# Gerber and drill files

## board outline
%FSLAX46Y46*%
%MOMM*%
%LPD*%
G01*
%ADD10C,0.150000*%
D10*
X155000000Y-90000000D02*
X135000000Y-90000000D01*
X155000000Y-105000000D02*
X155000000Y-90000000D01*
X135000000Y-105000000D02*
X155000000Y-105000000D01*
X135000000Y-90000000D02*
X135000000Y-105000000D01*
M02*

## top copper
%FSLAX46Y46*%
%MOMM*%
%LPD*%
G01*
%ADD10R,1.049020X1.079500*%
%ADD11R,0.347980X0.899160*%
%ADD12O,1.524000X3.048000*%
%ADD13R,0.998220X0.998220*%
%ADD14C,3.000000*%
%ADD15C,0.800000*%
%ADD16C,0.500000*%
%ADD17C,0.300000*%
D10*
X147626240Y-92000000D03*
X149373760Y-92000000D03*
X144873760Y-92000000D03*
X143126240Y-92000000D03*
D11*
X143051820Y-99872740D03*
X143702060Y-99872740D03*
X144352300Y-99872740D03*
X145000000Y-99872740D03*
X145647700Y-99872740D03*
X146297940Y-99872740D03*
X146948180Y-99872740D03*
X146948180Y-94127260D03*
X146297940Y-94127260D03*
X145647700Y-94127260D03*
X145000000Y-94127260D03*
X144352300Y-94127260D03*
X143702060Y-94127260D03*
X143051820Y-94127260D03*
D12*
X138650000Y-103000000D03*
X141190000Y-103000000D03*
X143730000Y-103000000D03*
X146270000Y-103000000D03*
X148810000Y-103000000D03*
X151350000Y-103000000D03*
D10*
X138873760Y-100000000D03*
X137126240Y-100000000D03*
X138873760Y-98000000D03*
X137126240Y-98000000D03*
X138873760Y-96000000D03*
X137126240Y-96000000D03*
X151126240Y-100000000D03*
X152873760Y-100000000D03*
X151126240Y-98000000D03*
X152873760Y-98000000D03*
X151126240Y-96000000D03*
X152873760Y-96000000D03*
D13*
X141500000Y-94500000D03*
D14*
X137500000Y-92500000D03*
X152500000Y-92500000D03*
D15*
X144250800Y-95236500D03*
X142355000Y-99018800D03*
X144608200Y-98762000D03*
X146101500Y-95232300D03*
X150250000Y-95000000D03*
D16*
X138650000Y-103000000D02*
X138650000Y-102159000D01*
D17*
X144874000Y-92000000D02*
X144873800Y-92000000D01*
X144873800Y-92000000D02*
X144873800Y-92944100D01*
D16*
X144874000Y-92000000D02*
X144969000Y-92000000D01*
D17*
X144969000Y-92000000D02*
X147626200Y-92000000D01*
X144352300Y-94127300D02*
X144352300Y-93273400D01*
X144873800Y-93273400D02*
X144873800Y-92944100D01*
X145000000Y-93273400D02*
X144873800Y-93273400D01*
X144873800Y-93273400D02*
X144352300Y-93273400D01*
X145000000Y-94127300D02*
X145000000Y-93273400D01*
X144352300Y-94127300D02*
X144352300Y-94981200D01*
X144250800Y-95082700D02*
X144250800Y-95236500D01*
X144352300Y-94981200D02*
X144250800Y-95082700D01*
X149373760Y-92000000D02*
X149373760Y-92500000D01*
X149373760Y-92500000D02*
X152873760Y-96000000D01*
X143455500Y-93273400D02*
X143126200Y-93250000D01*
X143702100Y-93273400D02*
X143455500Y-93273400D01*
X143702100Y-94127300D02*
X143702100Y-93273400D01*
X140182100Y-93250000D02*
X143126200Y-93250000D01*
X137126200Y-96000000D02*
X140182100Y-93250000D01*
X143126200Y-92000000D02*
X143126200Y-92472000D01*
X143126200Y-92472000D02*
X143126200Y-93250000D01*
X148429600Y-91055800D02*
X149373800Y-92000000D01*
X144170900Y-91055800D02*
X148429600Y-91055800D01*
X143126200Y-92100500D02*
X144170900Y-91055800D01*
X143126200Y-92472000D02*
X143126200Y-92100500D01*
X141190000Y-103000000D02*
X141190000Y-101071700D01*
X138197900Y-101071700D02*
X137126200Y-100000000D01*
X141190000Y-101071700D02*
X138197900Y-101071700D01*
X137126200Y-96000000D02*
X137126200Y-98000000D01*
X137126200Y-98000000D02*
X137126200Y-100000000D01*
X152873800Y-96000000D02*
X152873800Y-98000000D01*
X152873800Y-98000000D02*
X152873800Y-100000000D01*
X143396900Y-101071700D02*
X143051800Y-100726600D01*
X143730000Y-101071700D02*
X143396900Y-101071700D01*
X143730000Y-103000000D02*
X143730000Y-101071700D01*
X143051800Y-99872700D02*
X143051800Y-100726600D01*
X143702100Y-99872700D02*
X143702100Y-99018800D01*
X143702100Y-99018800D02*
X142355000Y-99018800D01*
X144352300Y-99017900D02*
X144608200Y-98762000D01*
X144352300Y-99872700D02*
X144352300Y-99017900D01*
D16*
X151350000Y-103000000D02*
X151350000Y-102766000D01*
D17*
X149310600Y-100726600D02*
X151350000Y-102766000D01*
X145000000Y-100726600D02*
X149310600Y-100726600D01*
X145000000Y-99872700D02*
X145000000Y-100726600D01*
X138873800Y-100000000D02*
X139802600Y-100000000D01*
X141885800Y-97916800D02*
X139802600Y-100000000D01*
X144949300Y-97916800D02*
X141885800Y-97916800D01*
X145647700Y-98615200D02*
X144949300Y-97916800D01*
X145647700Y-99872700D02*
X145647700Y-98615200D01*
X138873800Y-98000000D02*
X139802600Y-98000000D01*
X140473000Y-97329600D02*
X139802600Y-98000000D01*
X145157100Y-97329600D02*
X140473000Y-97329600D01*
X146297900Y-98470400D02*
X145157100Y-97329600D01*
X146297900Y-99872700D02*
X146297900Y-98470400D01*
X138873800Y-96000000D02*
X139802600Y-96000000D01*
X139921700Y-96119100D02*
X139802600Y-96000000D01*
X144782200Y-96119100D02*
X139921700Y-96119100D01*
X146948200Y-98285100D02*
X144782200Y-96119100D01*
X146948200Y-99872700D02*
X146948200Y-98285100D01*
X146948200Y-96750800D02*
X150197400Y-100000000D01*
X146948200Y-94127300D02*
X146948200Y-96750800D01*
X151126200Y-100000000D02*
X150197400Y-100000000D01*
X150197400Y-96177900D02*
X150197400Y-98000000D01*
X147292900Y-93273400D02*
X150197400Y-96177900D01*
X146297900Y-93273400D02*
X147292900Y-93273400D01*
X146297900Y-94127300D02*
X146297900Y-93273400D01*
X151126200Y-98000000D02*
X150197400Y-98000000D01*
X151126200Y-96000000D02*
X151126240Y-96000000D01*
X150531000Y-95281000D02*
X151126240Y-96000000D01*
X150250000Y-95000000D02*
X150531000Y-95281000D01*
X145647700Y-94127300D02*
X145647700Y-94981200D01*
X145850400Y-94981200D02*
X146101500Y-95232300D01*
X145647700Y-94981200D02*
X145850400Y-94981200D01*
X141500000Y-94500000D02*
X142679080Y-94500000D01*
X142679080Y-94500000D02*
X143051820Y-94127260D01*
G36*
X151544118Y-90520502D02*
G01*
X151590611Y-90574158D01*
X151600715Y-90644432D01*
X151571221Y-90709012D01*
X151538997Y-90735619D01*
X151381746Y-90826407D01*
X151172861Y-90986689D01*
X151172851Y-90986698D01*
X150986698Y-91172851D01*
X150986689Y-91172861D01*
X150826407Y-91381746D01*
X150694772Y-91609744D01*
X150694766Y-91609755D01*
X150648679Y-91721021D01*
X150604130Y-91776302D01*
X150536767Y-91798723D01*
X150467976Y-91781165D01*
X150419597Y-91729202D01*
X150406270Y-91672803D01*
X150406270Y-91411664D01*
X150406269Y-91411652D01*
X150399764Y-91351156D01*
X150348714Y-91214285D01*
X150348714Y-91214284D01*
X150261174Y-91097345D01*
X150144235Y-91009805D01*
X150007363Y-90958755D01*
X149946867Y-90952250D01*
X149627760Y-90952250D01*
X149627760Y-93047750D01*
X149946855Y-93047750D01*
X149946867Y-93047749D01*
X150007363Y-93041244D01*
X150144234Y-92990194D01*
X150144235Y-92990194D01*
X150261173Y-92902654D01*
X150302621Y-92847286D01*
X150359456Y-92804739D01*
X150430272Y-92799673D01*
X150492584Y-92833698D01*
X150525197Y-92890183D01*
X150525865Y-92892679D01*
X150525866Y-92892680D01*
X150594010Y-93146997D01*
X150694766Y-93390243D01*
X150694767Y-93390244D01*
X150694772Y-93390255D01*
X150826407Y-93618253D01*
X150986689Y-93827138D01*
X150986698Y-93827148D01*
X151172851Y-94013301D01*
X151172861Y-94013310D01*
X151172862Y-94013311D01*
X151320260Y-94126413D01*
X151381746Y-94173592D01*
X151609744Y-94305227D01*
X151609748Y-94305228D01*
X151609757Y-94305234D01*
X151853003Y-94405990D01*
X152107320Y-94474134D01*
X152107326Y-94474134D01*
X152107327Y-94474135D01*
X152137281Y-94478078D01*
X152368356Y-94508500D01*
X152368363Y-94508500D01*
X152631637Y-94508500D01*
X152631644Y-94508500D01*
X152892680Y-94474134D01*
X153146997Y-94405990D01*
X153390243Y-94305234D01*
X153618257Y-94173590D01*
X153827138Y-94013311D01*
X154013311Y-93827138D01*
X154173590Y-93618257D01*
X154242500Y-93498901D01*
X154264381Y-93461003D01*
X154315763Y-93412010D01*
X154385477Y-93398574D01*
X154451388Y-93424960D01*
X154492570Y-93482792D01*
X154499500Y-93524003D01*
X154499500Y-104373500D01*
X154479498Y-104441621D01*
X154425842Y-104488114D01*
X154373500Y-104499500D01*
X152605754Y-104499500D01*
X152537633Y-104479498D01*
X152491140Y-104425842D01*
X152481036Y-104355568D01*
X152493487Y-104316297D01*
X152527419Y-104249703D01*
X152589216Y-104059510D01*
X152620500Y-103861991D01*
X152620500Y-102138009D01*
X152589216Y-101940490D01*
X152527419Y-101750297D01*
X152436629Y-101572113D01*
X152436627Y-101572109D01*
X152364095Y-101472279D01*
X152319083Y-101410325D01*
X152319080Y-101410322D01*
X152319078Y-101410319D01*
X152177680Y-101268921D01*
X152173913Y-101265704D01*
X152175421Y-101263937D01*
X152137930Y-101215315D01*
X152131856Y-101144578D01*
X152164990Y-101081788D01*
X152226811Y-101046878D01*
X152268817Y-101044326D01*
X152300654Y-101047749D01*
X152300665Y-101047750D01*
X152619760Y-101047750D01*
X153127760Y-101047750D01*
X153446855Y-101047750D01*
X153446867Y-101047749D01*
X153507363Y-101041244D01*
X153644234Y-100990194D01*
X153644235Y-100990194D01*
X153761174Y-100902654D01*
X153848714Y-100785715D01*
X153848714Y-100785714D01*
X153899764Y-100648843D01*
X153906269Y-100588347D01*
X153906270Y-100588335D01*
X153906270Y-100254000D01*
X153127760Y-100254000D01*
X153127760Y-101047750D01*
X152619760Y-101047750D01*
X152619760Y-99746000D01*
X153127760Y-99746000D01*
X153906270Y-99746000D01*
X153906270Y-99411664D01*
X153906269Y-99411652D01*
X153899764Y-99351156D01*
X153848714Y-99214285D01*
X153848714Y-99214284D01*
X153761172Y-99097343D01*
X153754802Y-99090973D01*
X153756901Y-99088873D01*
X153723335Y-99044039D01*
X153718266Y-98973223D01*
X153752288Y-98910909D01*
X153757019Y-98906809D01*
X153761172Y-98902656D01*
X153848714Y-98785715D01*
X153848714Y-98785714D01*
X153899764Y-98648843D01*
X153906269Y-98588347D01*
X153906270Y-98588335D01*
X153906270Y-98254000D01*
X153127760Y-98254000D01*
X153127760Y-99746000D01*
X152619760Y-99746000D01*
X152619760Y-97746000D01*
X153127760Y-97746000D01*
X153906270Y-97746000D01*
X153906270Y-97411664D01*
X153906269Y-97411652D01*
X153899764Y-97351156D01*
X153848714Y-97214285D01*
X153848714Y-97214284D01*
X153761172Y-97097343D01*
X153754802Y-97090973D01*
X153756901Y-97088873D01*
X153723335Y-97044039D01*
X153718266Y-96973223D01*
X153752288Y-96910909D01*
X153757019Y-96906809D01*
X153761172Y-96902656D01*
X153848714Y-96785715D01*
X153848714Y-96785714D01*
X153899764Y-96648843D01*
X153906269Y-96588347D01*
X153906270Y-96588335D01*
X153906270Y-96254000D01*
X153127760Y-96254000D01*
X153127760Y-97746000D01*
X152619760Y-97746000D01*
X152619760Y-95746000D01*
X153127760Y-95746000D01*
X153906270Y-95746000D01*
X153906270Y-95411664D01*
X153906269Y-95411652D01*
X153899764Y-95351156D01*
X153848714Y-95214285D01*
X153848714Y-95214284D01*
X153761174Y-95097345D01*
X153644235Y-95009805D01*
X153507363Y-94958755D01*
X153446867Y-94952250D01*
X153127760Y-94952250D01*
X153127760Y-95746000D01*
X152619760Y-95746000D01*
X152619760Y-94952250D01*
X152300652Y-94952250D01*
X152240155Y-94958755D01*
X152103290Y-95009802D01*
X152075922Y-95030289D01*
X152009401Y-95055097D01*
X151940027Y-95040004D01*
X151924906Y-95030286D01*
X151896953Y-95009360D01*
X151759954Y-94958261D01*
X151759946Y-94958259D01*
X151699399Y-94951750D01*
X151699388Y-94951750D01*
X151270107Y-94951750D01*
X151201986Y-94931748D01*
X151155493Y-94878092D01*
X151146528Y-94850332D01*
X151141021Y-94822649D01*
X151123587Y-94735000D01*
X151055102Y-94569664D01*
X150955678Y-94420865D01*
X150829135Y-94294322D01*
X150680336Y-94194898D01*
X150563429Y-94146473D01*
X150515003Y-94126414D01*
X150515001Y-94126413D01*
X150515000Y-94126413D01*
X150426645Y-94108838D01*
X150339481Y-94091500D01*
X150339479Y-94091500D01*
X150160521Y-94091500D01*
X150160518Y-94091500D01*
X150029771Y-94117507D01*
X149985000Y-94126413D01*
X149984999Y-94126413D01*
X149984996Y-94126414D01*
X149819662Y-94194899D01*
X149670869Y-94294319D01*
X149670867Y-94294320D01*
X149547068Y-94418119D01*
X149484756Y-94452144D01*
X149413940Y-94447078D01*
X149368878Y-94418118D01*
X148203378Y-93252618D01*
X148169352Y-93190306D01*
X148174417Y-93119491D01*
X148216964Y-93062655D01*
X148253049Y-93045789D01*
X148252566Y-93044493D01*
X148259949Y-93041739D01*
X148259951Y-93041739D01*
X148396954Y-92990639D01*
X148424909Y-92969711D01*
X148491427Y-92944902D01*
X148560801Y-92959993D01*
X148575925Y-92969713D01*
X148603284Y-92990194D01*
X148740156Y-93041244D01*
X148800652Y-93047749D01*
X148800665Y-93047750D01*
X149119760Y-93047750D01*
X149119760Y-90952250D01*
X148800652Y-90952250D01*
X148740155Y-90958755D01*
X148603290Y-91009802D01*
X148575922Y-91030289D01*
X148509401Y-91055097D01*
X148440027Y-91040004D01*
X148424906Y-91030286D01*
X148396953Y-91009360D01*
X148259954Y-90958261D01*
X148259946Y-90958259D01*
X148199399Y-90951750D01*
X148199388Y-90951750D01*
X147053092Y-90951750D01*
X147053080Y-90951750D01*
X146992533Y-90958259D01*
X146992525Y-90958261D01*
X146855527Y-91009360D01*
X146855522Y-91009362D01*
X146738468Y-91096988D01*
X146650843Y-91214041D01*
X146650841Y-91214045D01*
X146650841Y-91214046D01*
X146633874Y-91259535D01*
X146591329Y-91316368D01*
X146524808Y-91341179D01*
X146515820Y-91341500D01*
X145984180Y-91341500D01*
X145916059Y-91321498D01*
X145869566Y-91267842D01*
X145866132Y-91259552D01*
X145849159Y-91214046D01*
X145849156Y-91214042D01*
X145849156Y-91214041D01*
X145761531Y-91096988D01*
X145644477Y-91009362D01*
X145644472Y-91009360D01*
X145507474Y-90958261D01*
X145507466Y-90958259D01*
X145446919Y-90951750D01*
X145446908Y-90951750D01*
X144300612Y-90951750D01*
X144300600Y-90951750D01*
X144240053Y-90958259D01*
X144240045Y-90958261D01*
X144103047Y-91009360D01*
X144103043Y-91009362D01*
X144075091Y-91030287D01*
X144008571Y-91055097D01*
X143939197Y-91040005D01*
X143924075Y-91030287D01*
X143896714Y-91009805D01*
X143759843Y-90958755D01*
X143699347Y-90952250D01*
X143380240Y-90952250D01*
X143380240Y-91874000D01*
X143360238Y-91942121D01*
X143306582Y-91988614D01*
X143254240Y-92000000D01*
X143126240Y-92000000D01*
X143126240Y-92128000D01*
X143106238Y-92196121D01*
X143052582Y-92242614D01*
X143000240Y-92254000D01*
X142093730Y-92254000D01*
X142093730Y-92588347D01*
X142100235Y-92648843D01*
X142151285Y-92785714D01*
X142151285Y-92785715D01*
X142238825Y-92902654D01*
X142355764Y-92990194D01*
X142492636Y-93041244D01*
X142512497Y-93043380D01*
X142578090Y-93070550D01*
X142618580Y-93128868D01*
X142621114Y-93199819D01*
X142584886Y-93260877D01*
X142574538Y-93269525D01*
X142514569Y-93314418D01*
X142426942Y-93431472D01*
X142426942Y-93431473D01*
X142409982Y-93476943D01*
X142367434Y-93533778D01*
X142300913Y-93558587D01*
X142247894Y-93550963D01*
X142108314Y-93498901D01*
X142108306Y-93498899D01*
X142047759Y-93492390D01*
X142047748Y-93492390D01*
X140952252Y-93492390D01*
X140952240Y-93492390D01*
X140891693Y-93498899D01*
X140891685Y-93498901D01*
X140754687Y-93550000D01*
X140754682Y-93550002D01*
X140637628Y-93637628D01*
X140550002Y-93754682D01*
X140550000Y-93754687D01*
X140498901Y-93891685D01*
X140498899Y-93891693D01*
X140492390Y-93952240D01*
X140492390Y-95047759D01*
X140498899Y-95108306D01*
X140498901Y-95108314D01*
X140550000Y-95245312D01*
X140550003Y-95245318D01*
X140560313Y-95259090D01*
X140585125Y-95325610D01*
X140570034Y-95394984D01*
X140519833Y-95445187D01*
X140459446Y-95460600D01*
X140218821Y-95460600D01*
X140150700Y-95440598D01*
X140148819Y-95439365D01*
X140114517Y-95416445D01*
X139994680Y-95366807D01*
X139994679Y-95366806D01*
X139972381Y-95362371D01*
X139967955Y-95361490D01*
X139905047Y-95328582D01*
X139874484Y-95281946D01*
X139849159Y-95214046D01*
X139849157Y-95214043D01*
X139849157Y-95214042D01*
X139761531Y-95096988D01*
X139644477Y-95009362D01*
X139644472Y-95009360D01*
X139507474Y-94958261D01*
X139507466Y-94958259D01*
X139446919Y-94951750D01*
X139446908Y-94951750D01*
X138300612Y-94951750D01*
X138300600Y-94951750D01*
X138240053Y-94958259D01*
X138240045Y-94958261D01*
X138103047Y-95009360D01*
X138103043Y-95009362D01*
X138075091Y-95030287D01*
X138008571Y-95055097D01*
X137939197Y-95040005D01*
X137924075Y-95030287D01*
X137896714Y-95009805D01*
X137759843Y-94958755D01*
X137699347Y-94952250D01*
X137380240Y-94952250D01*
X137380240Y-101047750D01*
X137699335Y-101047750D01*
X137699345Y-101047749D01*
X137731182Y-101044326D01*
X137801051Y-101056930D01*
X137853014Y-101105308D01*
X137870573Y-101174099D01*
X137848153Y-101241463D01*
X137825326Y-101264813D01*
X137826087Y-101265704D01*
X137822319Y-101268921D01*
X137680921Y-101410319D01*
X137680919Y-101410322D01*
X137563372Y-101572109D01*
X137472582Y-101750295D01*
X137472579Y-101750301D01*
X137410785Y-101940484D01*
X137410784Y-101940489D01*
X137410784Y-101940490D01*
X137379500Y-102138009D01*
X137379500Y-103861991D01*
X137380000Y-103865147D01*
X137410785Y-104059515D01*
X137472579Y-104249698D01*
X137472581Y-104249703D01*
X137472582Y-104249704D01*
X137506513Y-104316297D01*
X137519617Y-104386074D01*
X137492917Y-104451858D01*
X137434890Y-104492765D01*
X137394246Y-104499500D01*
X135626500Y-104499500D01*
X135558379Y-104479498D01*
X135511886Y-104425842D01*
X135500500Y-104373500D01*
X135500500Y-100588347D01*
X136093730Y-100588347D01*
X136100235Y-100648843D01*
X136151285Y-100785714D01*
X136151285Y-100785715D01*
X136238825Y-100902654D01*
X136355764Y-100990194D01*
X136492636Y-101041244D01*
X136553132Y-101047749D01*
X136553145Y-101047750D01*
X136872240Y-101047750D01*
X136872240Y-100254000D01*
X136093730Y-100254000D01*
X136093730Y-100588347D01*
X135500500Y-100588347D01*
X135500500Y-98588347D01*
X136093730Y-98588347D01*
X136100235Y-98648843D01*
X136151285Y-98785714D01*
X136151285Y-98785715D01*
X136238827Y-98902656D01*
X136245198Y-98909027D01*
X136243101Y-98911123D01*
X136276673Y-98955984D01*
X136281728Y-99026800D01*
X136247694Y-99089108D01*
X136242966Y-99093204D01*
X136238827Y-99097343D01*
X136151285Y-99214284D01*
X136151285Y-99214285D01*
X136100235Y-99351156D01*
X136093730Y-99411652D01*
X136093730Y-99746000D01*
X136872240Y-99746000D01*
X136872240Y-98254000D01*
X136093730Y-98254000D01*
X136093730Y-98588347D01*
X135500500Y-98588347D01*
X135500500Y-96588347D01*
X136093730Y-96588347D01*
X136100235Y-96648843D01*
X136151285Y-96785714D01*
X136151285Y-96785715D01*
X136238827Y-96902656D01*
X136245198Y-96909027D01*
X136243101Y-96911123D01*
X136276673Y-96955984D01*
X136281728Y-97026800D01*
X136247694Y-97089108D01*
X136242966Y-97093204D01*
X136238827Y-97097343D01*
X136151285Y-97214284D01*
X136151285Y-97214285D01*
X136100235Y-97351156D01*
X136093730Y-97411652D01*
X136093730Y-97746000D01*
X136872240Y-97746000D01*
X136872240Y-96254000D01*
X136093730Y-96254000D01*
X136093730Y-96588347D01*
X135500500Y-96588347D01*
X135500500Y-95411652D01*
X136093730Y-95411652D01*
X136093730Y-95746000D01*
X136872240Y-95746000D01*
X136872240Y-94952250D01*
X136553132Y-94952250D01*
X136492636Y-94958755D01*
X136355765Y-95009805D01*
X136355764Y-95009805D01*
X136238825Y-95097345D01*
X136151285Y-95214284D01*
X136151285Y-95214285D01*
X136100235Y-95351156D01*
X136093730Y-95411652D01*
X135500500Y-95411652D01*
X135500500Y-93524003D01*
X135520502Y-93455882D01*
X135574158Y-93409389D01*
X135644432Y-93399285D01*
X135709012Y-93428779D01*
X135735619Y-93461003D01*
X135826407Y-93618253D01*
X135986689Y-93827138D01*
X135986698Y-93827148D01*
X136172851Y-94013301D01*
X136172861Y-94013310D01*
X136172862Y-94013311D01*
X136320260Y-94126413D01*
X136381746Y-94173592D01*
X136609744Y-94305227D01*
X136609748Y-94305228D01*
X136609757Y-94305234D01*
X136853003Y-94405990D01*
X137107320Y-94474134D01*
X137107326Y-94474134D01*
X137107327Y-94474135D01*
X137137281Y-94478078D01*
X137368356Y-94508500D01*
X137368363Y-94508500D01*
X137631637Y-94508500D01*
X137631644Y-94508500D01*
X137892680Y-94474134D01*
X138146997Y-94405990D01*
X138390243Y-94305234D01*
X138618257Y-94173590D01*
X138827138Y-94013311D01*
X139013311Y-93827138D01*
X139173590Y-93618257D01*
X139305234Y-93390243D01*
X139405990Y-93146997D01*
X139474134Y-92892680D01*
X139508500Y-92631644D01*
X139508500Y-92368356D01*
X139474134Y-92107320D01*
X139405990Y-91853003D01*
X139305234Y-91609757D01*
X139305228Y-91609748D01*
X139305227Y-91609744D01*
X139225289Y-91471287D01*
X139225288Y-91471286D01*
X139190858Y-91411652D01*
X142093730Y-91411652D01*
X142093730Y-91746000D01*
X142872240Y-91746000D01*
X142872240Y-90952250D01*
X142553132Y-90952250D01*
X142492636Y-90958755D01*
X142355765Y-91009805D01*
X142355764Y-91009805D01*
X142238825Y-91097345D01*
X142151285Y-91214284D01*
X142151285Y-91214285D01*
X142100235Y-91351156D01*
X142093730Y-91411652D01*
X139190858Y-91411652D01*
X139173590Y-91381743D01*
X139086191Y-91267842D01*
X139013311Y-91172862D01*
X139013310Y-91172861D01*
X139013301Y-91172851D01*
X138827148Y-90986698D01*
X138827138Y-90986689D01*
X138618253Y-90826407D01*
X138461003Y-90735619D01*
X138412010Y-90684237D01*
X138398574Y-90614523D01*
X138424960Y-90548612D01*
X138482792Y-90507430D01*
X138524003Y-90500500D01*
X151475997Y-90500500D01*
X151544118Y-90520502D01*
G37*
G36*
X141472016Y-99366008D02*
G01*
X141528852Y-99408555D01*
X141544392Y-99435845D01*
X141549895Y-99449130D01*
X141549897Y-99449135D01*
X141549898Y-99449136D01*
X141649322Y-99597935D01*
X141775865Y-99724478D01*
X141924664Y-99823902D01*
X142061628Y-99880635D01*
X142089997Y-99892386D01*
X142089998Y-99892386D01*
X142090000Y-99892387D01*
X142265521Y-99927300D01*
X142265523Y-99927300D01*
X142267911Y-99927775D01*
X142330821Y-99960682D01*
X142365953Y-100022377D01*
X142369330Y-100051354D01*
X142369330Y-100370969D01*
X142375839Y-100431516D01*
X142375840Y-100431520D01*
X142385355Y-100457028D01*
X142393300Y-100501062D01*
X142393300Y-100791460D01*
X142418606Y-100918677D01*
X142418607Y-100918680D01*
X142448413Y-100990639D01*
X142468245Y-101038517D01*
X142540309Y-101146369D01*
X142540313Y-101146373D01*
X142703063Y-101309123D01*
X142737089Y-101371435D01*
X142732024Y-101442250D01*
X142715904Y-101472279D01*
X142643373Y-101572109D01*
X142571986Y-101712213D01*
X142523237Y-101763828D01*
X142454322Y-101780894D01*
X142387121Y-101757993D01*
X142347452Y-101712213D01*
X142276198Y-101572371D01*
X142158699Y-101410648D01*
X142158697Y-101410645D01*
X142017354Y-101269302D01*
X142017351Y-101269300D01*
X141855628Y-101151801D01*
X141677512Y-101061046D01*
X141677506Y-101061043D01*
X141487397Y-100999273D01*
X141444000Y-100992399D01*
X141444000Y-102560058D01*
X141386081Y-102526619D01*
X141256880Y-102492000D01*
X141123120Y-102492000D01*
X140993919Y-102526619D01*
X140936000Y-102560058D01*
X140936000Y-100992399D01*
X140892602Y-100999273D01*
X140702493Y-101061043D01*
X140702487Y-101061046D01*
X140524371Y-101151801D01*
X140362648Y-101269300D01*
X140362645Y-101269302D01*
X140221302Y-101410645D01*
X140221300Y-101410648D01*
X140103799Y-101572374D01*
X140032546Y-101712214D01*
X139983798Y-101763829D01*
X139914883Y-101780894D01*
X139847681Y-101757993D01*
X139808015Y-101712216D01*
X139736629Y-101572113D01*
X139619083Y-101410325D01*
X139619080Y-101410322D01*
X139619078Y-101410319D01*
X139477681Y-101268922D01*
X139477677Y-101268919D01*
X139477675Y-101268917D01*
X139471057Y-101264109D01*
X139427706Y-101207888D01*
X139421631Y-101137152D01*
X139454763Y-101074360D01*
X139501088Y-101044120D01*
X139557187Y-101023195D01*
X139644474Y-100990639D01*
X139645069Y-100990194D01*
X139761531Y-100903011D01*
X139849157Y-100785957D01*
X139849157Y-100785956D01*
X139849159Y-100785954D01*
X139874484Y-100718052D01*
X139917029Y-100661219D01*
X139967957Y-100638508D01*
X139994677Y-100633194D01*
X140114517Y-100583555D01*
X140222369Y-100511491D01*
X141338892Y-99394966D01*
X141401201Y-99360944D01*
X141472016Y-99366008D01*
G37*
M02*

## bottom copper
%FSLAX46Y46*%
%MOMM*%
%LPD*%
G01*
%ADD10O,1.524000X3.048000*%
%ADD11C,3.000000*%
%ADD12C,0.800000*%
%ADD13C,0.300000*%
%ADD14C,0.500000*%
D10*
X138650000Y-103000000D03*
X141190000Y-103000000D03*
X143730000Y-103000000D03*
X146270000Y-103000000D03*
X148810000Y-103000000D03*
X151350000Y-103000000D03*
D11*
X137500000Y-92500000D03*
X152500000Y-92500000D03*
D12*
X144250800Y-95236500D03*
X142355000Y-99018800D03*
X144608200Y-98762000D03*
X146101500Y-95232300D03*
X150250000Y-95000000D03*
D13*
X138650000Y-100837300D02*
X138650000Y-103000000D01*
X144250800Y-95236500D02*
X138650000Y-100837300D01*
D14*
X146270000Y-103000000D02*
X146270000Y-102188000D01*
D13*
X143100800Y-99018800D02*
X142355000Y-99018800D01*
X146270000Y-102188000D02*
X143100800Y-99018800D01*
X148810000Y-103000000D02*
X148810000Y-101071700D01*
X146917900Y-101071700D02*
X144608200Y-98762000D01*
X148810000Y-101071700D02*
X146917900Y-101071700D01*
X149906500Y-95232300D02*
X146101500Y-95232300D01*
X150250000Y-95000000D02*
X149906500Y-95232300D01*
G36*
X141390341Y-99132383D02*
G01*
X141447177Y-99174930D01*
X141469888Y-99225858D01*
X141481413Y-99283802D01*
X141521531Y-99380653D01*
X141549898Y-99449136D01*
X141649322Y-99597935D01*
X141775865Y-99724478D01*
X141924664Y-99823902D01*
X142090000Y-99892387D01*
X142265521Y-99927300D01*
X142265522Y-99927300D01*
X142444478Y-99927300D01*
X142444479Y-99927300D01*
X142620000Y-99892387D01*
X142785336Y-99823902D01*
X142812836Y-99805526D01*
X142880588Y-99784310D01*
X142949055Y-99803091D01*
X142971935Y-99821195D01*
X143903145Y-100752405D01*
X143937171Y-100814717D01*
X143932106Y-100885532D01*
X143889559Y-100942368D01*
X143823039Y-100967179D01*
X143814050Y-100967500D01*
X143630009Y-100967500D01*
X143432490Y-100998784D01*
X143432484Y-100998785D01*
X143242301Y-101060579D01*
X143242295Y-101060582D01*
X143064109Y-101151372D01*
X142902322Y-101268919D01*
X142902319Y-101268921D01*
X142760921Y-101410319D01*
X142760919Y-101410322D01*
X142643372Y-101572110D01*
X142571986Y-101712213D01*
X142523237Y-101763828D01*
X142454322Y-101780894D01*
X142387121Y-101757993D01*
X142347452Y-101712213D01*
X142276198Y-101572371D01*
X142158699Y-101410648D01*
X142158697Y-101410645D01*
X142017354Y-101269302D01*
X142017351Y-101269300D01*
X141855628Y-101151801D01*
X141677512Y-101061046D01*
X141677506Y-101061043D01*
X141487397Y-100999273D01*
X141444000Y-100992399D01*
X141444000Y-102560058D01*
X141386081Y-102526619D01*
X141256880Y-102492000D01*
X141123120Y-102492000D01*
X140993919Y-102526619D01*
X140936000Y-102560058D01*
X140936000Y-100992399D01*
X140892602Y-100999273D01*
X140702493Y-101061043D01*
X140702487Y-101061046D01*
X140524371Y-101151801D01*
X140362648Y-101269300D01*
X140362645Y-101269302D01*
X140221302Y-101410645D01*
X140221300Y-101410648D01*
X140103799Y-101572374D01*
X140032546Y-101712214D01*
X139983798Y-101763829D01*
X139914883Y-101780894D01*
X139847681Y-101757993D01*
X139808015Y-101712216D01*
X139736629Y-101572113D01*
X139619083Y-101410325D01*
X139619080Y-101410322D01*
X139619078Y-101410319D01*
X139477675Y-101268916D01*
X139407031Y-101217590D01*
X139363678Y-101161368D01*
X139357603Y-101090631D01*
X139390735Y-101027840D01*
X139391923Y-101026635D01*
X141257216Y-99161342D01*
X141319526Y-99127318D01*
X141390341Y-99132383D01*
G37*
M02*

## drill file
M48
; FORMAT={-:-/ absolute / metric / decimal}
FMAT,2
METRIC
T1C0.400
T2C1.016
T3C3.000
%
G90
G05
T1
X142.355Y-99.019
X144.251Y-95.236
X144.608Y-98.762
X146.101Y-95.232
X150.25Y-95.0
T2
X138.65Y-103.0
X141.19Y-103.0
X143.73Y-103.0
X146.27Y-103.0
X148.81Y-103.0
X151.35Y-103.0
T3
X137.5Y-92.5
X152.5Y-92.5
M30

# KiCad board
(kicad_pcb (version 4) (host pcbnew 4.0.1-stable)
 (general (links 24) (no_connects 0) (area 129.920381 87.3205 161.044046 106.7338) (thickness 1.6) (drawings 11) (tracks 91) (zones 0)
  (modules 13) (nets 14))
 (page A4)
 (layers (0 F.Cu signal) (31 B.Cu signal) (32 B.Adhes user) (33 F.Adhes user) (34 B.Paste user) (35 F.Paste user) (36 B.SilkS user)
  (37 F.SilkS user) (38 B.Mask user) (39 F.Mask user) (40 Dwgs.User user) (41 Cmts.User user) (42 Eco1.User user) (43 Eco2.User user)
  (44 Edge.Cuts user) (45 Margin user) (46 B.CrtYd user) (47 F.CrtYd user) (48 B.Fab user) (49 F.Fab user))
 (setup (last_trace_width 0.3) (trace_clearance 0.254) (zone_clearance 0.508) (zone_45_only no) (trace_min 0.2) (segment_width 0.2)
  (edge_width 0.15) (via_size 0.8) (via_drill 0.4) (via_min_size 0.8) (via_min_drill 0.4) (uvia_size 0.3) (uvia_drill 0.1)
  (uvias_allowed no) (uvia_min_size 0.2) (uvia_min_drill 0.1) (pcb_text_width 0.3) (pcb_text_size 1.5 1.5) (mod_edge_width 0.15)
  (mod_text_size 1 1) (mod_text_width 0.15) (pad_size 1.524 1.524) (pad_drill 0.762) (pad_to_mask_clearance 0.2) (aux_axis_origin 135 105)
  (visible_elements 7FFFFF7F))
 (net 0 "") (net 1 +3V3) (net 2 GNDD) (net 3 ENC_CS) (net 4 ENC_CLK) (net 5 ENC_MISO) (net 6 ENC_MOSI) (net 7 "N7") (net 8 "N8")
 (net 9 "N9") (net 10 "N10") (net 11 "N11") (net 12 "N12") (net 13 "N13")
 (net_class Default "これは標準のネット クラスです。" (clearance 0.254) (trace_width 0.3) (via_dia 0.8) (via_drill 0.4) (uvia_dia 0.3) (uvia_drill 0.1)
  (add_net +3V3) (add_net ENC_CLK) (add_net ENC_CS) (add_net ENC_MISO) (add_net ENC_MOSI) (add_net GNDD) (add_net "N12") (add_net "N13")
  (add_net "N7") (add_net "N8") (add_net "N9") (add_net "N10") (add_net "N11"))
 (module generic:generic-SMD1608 (layer F.Cu) (at 148.5 92)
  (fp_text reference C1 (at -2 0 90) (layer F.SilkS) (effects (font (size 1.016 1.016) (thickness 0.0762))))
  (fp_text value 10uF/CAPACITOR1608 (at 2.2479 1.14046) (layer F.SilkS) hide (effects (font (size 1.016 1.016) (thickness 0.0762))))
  (pad 1 smd rect (at -0.87376 0) (size 1.04902 1.0795) (layers F.Cu F.Paste F.Mask) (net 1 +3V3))
  (pad 2 smd rect (at 0.87376 0) (size 1.04902 1.0795) (layers F.Cu F.Paste F.Mask) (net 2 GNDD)))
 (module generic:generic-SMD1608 (layer F.Cu) (at 144 92 180)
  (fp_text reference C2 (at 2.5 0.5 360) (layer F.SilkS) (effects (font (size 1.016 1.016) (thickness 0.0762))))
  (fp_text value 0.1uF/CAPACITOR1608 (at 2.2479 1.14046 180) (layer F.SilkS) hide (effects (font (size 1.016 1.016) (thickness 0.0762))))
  (pad 1 smd rect (at -0.87376 0 180) (size 1.04902 1.0795) (layers F.Cu F.Paste F.Mask) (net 1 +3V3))
  (pad 2 smd rect (at 0.87376 0 180) (size 1.04902 1.0795) (layers F.Cu F.Paste F.Mask) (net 2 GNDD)))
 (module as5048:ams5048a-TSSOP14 (layer F.Cu) (at 145 97 90)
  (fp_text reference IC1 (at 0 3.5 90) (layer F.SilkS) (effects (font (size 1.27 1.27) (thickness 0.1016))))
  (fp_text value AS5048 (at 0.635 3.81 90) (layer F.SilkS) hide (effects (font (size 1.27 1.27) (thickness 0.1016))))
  (pad 1 smd rect (at -2.87274 -1.94818 90) (size 0.89916 0.34798) (layers F.Cu F.Paste F.Mask) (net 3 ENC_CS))
  (pad 2 smd rect (at -2.87274 -1.29794 90) (size 0.89916 0.34798) (layers F.Cu F.Paste F.Mask) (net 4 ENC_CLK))
  (pad 3 smd rect (at -2.87274 -0.6477 90) (size 0.89916 0.34798) (layers F.Cu F.Paste F.Mask) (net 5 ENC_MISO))
  (pad 4 smd rect (at -2.87274 0 90) (size 0.89916 0.34798) (layers F.Cu F.Paste F.Mask) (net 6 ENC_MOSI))
  (pad 5 smd rect (at -2.87274 0.6477 90) (size 0.89916 0.34798) (layers F.Cu F.Paste F.Mask) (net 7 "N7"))
  (pad 6 smd rect (at -2.87274 1.29794 90) (size 0.89916 0.34798) (layers F.Cu F.Paste F.Mask) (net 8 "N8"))
  (pad 7 smd rect (at -2.87274 1.94818 90) (size 0.89916 0.34798) (layers F.Cu F.Paste F.Mask) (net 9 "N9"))
  (pad 8 smd rect (at 2.87274 1.94818 90) (size 0.89916 0.34798) (layers F.Cu F.Paste F.Mask) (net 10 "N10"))
  (pad 9 smd rect (at 2.87274 1.29794 90) (size 0.89916 0.34798) (layers F.Cu F.Paste F.Mask) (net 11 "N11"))
  (pad 10 smd rect (at 2.87274 0.6477 90) (size 0.89916 0.34798) (layers F.Cu F.Paste F.Mask) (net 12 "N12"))
  (pad 11 smd rect (at 2.87274 0 90) (size 0.89916 0.34798) (layers F.Cu F.Paste F.Mask) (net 1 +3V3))
  (pad 12 smd rect (at 2.87274 -0.6477 90) (size 0.89916 0.34798) (layers F.Cu F.Paste F.Mask) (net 1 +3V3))
  (pad 13 smd rect (at 2.87274 -1.29794 90) (size 0.89916 0.34798) (layers F.Cu F.Paste F.Mask) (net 2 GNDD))
  (pad 14 smd rect (at 2.87274 -1.94818 90) (size 0.89916 0.34798) (layers F.Cu F.Paste F.Mask) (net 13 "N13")))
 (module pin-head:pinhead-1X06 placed (layer F.Cu) (at 145 103)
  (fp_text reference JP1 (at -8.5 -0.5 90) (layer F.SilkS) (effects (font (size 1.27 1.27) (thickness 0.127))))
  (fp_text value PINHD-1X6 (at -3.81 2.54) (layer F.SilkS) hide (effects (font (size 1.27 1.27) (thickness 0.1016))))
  (pad 1 thru_hole oval (at -6.35 0 180) (size 1.524 3.048) (drill 1.016) (layers *.Cu F.Paste F.SilkS F.Mask) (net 1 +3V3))
  (pad 2 thru_hole oval (at -3.81 0 180) (size 1.524 3.048) (drill 1.016) (layers *.Cu F.Paste F.SilkS F.Mask) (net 2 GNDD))
  (pad 3 thru_hole oval (at -1.27 0 180) (size 1.524 3.048) (drill 1.016) (layers *.Cu F.Paste F.SilkS F.Mask) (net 3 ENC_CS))
  (pad 4 thru_hole oval (at 1.27 0 180) (size 1.524 3.048) (drill 1.016) (layers *.Cu F.Paste F.SilkS F.Mask) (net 4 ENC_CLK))
  (pad 5 thru_hole oval (at 3.81 0 180) (size 1.524 3.048) (drill 1.016) (layers *.Cu F.Paste F.SilkS F.Mask) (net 5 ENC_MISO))
  (pad 6 thru_hole oval (at 6.35 0 180) (size 1.524 3.048) (drill 1.016) (layers *.Cu F.Paste F.SilkS F.Mask) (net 6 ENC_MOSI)))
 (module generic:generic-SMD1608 (layer F.Cu) (at 138 100 180)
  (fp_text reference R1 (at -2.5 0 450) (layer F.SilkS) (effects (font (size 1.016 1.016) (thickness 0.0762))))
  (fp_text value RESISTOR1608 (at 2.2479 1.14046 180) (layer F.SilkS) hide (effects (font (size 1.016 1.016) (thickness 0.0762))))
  (pad 1 smd rect (at -0.87376 0 180) (size 1.04902 1.0795) (layers F.Cu F.Paste F.Mask) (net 7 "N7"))
  (pad 2 smd rect (at 0.87376 0 180) (size 1.04902 1.0795) (layers F.Cu F.Paste F.Mask) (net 2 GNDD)))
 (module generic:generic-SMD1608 (layer F.Cu) (at 138 98 180)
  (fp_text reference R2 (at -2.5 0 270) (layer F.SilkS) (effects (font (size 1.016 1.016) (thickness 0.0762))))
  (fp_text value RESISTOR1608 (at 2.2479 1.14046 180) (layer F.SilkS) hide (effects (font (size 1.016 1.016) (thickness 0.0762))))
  (pad 1 smd rect (at -0.87376 0 180) (size 1.04902 1.0795) (layers F.Cu F.Paste F.Mask) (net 8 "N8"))
  (pad 2 smd rect (at 0.87376 0 180) (size 1.04902 1.0795) (layers F.Cu F.Paste F.Mask) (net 2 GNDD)))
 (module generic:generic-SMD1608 (layer F.Cu) (at 138 96 180)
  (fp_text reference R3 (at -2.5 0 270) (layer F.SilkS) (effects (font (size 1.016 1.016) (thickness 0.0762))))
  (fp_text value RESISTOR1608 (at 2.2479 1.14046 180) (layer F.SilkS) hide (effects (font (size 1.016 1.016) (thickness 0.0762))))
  (pad 1 smd rect (at -0.87376 0 180) (size 1.04902 1.0795) (layers F.Cu F.Paste F.Mask) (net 9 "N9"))
  (pad 2 smd rect (at 0.87376 0 180) (size 1.04902 1.0795) (layers F.Cu F.Paste F.Mask) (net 2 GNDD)))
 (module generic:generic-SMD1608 (layer F.Cu) (at 152 100)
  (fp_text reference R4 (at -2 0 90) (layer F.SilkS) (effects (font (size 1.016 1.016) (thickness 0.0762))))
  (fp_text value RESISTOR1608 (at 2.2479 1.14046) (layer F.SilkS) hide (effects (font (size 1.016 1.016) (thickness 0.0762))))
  (pad 1 smd rect (at -0.87376 0) (size 1.04902 1.0795) (layers F.Cu F.Paste F.Mask) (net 10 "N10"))
  (pad 2 smd rect (at 0.87376 0) (size 1.04902 1.0795) (layers F.Cu F.Paste F.Mask) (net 2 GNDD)))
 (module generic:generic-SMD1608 (layer F.Cu) (at 152 98)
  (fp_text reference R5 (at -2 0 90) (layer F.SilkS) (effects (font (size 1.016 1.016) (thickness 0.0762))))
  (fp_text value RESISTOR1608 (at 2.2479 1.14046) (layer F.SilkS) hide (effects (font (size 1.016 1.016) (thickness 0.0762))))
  (pad 1 smd rect (at -0.87376 0) (size 1.04902 1.0795) (layers F.Cu F.Paste F.Mask) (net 11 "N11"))
  (pad 2 smd rect (at 0.87376 0) (size 1.04902 1.0795) (layers F.Cu F.Paste F.Mask) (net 2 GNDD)))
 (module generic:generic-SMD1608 (layer F.Cu) (at 152 96)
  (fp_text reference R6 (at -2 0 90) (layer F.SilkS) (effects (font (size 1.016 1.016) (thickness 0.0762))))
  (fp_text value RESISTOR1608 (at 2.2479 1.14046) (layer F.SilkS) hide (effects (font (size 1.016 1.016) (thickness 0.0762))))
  (pad 1 smd rect (at -0.87376 0) (size 1.04902 1.0795) (layers F.Cu F.Paste F.Mask) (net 12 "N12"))
  (pad 2 smd rect (at 0.87376 0) (size 1.04902 1.0795) (layers F.Cu F.Paste F.Mask) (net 2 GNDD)))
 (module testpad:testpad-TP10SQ (layer F.Cu) (at 141 94.5)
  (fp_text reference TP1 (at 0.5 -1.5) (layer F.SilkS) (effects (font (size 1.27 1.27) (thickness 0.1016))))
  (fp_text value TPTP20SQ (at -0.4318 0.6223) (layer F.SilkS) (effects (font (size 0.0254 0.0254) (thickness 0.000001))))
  (pad TP smd rect (at 0.5 0) (size 0.99822 0.99822) (layers F.Cu F.Paste F.Mask) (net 13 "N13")))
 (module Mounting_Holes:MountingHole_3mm (layer F.Cu) (at 137.5 92.5)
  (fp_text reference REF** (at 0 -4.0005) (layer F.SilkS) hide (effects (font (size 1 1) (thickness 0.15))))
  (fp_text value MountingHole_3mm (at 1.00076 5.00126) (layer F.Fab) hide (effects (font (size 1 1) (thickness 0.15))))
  (pad 1 thru_hole circle (at 0 0) (size 3 3) (drill 3) (layers)))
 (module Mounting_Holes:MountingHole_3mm (layer F.Cu) (at 152.5 92.5)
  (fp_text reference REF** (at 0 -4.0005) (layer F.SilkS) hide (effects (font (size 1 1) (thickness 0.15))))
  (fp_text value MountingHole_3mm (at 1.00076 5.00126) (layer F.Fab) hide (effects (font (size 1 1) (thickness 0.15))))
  (pad 1 thru_hole circle (at 0 0) (size 3 3) (drill 3) (layers)))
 (gr_line (start 155 90) (end 135 90) (angle 90) (layer Edge.Cuts) (width 0.15))
 (gr_line (start 155 105) (end 155 90) (angle 90) (layer Edge.Cuts) (width 0.15))
 (gr_line (start 135 105) (end 155 105) (angle 90) (layer Edge.Cuts) (width 0.15))
 (gr_line (start 135 90) (end 135 105) (angle 90) (layer Edge.Cuts) (width 0.15))
 (via (at 144.2508 95.2365) (size 0.8) (layers F.Cu B.Cu) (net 1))
 (segment (start 138.65 103) (end 138.65 102.159) (width 0.5) (layer F.Cu) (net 1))
 (segment (start 144.874 92) (end 144.8738 92) (width 0.3) (layer F.Cu) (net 1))
 (segment (start 144.8738 92) (end 144.8738 92.9441) (width 0.3) (layer F.Cu) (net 1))
 (segment (start 144.874 92) (end 144.969 92) (width 0.5) (layer F.Cu) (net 1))
 (segment (start 144.969 92) (end 147.6262 92) (width 0.3) (layer F.Cu) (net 1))
 (segment (start 144.3523 94.1273) (end 144.3523 93.2734) (width 0.3) (layer F.Cu) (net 1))
 (segment (start 144.8738 93.2734) (end 144.8738 92.9441) (width 0.3) (layer F.Cu) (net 1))
 (segment (start 145 93.2734) (end 144.8738 93.2734) (width 0.3) (layer F.Cu) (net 1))
 (segment (start 144.8738 93.2734) (end 144.3523 93.2734) (width 0.3) (layer F.Cu) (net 1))
 (segment (start 145 94.1273) (end 145 93.2734) (width 0.3) (layer F.Cu) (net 1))
 (segment (start 144.3523 94.1273) (end 144.3523 94.9812) (width 0.3) (layer F.Cu) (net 1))
 (segment (start 144.2508 95.0827) (end 144.2508 95.2365) (width 0.3) (layer F.Cu) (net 1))
 (segment (start 144.3523 94.9812) (end 144.2508 95.0827) (width 0.3) (layer F.Cu) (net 1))
 (segment (start 138.65 100.8373) (end 138.65 103) (width 0.3) (layer B.Cu) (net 1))
 (segment (start 144.2508 95.2365) (end 138.65 100.8373) (width 0.3) (layer B.Cu) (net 1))
 (segment (start 149.37376 92) (end 149.37376 92.5) (width 0.3) (layer F.Cu) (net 2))
 (segment (start 149.37376 92.5) (end 152.87376 96) (width 0.3) (layer F.Cu) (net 2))
 (segment (start 143.4555 93.2734) (end 143.1262 93.25) (width 0.3) (layer F.Cu) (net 2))
 (segment (start 143.7021 93.2734) (end 143.4555 93.2734) (width 0.3) (layer F.Cu) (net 2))
 (segment (start 143.7021 94.1273) (end 143.7021 93.2734) (width 0.3) (layer F.Cu) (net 2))
 (segment (start 140.1821 93.25) (end 143.1262 93.25) (width 0.3) (layer F.Cu) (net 2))
 (segment (start 137.1262 96) (end 140.1821 93.25) (width 0.3) (layer F.Cu) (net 2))
 (segment (start 143.1262 92) (end 143.1262 92.472) (width 0.3) (layer F.Cu) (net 2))
 (segment (start 143.1262 92.472) (end 143.1262 93.25) (width 0.3) (layer F.Cu) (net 2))
 (segment (start 148.4296 91.0558) (end 149.3738 92) (width 0.3) (layer F.Cu) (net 2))
 (segment (start 144.1709 91.0558) (end 148.4296 91.0558) (width 0.3) (layer F.Cu) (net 2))
 (segment (start 143.1262 92.1005) (end 144.1709 91.0558) (width 0.3) (layer F.Cu) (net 2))
 (segment (start 143.1262 92.472) (end 143.1262 92.1005) (width 0.3) (layer F.Cu) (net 2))
 (segment (start 141.19 103) (end 141.19 101.0717) (width 0.3) (layer F.Cu) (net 2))
 (segment (start 138.1979 101.0717) (end 137.1262 100) (width 0.3) (layer F.Cu) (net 2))
 (segment (start 141.19 101.0717) (end 138.1979 101.0717) (width 0.3) (layer F.Cu) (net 2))
 (segment (start 137.1262 96) (end 137.1262 98) (width 0.3) (layer F.Cu) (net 2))
 (segment (start 137.1262 98) (end 137.1262 100) (width 0.3) (layer F.Cu) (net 2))
 (segment (start 152.8738 96) (end 152.8738 98) (width 0.3) (layer F.Cu) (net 2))
 (segment (start 152.8738 98) (end 152.8738 100) (width 0.3) (layer F.Cu) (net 2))
 (segment (start 143.3969 101.0717) (end 143.0518 100.7266) (width 0.3) (layer F.Cu) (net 3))
 (segment (start 143.73 101.0717) (end 143.3969 101.0717) (width 0.3) (layer F.Cu) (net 3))
 (segment (start 143.73 103) (end 143.73 101.0717) (width 0.3) (layer F.Cu) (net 3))
 (segment (start 143.0518 99.8727) (end 143.0518 100.7266) (width 0.3) (layer F.Cu) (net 3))
 (via (at 142.355 99.0188) (size 0.8) (layers F.Cu B.Cu) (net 4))
 (segment (start 146.27 103) (end 146.27 102.188) (width 0.5) (layer B.Cu) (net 4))
 (segment (start 143.7021 99.8727) (end 143.7021 99.0188) (width 0.3) (layer F.Cu) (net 4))
 (segment (start 143.1008 99.0188) (end 142.355 99.0188) (width 0.3) (layer B.Cu) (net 4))
 (segment (start 146.27 102.188) (end 143.1008 99.0188) (width 0.3) (layer B.Cu) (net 4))
 (segment (start 143.7021 99.0188) (end 142.355 99.0188) (width 0.3) (layer F.Cu) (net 4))
 (via (at 144.6082 98.762) (size 0.8) (layers F.Cu B.Cu) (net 5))
 (segment (start 148.81 103) (end 148.81 101.0717) (width 0.3) (layer B.Cu) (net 5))
 (segment (start 144.3523 99.0179) (end 144.6082 98.762) (width 0.3) (layer F.Cu) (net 5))
 (segment (start 144.3523 99.8727) (end 144.3523 99.0179) (width 0.3) (layer F.Cu) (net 5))
 (segment (start 146.9179 101.0717) (end 144.6082 98.762) (width 0.3) (layer B.Cu) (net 5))
 (segment (start 148.81 101.0717) (end 146.9179 101.0717) (width 0.3) (layer B.Cu) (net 5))
 (segment (start 151.35 103) (end 151.35 102.766) (width 0.5) (layer F.Cu) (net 6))
 (segment (start 149.3106 100.7266) (end 151.35 102.766) (width 0.3) (layer F.Cu) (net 6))
 (segment (start 145 100.7266) (end 149.3106 100.7266) (width 0.3) (layer F.Cu) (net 6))
 (segment (start 145 99.8727) (end 145 100.7266) (width 0.3) (layer F.Cu) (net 6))
 (segment (start 138.8738 100) (end 139.8026 100) (width 0.3) (layer F.Cu) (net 7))
 (segment (start 141.8858 97.9168) (end 139.8026 100) (width 0.3) (layer F.Cu) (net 7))
 (segment (start 144.9493 97.9168) (end 141.8858 97.9168) (width 0.3) (layer F.Cu) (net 7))
 (segment (start 145.6477 98.6152) (end 144.9493 97.9168) (width 0.3) (layer F.Cu) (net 7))
 (segment (start 145.6477 99.8727) (end 145.6477 98.6152) (width 0.3) (layer F.Cu) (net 7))
 (segment (start 138.8738 98) (end 139.8026 98) (width 0.3) (layer F.Cu) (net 8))
 (segment (start 140.473 97.3296) (end 139.8026 98) (width 0.3) (layer F.Cu) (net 8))
 (segment (start 145.1571 97.3296) (end 140.473 97.3296) (width 0.3) (layer F.Cu) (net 8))
 (segment (start 146.2979 98.4704) (end 145.1571 97.3296) (width 0.3) (layer F.Cu) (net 8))
 (segment (start 146.2979 99.8727) (end 146.2979 98.4704) (width 0.3) (layer F.Cu) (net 8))
 (segment (start 138.8738 96) (end 139.8026 96) (width 0.3) (layer F.Cu) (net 9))
 (segment (start 139.9217 96.1191) (end 139.8026 96) (width 0.3) (layer F.Cu) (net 9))
 (segment (start 144.7822 96.1191) (end 139.9217 96.1191) (width 0.3) (layer F.Cu) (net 9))
 (segment (start 146.9482 98.2851) (end 144.7822 96.1191) (width 0.3) (layer F.Cu) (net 9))
 (segment (start 146.9482 99.8727) (end 146.9482 98.2851) (width 0.3) (layer F.Cu) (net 9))
 (segment (start 146.9482 96.7508) (end 150.1974 100) (width 0.3) (layer F.Cu) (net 10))
 (segment (start 146.9482 94.1273) (end 146.9482 96.7508) (width 0.3) (layer F.Cu) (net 10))
 (segment (start 151.1262 100) (end 150.1974 100) (width 0.3) (layer F.Cu) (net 10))
 (segment (start 150.1974 96.1779) (end 150.1974 98) (width 0.3) (layer F.Cu) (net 11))
 (segment (start 147.2929 93.2734) (end 150.1974 96.1779) (width 0.3) (layer F.Cu) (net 11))
 (segment (start 146.2979 93.2734) (end 147.2929 93.2734) (width 0.3) (layer F.Cu) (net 11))
 (segment (start 146.2979 94.1273) (end 146.2979 93.2734) (width 0.3) (layer F.Cu) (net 11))
 (segment (start 151.1262 98) (end 150.1974 98) (width 0.3) (layer F.Cu) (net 11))
 (via (at 146.1015 95.2323) (size 0.8) (layers F.Cu B.Cu) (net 12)) (via (at 150.25 95) (size 0.8) (layers F.Cu B.Cu) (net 12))
 (segment (start 151.1262 96) (end 151.12624 96) (width 0.3) (layer F.Cu) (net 12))
 (segment (start 150.531 95.281) (end 151.12624 96) (width 0.3) (layer F.Cu) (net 12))
 (segment (start 150.25 95) (end 150.531 95.281) (width 0.3) (layer F.Cu) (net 12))
 (segment (start 145.6477 94.1273) (end 145.6477 94.9812) (width 0.3) (layer F.Cu) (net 12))
 (segment (start 149.9065 95.2323) (end 146.1015 95.2323) (width 0.3) (layer B.Cu) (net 12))
 (segment (start 150.25 95) (end 149.9065 95.2323) (width 0.3) (layer B.Cu) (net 12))
 (segment (start 145.8504 94.9812) (end 146.1015 95.2323) (width 0.3) (layer F.Cu) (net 12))
 (segment (start 145.6477 94.9812) (end 145.8504 94.9812) (width 0.3) (layer F.Cu) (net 12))
 (segment (start 141.5 94.5) (end 142.67908 94.5) (width 0.3) (layer F.Cu) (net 13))
 (segment (start 142.67908 94.5) (end 143.05182 94.12726) (width 0.3) (layer F.Cu) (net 13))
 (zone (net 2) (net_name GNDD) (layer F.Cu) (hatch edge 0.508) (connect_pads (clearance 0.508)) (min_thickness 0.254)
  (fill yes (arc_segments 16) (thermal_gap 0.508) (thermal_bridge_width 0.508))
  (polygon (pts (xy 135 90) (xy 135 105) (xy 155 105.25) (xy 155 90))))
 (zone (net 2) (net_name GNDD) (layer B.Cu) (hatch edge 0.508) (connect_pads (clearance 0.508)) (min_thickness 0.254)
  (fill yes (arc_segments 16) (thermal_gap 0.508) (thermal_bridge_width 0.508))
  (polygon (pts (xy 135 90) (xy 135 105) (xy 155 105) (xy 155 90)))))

